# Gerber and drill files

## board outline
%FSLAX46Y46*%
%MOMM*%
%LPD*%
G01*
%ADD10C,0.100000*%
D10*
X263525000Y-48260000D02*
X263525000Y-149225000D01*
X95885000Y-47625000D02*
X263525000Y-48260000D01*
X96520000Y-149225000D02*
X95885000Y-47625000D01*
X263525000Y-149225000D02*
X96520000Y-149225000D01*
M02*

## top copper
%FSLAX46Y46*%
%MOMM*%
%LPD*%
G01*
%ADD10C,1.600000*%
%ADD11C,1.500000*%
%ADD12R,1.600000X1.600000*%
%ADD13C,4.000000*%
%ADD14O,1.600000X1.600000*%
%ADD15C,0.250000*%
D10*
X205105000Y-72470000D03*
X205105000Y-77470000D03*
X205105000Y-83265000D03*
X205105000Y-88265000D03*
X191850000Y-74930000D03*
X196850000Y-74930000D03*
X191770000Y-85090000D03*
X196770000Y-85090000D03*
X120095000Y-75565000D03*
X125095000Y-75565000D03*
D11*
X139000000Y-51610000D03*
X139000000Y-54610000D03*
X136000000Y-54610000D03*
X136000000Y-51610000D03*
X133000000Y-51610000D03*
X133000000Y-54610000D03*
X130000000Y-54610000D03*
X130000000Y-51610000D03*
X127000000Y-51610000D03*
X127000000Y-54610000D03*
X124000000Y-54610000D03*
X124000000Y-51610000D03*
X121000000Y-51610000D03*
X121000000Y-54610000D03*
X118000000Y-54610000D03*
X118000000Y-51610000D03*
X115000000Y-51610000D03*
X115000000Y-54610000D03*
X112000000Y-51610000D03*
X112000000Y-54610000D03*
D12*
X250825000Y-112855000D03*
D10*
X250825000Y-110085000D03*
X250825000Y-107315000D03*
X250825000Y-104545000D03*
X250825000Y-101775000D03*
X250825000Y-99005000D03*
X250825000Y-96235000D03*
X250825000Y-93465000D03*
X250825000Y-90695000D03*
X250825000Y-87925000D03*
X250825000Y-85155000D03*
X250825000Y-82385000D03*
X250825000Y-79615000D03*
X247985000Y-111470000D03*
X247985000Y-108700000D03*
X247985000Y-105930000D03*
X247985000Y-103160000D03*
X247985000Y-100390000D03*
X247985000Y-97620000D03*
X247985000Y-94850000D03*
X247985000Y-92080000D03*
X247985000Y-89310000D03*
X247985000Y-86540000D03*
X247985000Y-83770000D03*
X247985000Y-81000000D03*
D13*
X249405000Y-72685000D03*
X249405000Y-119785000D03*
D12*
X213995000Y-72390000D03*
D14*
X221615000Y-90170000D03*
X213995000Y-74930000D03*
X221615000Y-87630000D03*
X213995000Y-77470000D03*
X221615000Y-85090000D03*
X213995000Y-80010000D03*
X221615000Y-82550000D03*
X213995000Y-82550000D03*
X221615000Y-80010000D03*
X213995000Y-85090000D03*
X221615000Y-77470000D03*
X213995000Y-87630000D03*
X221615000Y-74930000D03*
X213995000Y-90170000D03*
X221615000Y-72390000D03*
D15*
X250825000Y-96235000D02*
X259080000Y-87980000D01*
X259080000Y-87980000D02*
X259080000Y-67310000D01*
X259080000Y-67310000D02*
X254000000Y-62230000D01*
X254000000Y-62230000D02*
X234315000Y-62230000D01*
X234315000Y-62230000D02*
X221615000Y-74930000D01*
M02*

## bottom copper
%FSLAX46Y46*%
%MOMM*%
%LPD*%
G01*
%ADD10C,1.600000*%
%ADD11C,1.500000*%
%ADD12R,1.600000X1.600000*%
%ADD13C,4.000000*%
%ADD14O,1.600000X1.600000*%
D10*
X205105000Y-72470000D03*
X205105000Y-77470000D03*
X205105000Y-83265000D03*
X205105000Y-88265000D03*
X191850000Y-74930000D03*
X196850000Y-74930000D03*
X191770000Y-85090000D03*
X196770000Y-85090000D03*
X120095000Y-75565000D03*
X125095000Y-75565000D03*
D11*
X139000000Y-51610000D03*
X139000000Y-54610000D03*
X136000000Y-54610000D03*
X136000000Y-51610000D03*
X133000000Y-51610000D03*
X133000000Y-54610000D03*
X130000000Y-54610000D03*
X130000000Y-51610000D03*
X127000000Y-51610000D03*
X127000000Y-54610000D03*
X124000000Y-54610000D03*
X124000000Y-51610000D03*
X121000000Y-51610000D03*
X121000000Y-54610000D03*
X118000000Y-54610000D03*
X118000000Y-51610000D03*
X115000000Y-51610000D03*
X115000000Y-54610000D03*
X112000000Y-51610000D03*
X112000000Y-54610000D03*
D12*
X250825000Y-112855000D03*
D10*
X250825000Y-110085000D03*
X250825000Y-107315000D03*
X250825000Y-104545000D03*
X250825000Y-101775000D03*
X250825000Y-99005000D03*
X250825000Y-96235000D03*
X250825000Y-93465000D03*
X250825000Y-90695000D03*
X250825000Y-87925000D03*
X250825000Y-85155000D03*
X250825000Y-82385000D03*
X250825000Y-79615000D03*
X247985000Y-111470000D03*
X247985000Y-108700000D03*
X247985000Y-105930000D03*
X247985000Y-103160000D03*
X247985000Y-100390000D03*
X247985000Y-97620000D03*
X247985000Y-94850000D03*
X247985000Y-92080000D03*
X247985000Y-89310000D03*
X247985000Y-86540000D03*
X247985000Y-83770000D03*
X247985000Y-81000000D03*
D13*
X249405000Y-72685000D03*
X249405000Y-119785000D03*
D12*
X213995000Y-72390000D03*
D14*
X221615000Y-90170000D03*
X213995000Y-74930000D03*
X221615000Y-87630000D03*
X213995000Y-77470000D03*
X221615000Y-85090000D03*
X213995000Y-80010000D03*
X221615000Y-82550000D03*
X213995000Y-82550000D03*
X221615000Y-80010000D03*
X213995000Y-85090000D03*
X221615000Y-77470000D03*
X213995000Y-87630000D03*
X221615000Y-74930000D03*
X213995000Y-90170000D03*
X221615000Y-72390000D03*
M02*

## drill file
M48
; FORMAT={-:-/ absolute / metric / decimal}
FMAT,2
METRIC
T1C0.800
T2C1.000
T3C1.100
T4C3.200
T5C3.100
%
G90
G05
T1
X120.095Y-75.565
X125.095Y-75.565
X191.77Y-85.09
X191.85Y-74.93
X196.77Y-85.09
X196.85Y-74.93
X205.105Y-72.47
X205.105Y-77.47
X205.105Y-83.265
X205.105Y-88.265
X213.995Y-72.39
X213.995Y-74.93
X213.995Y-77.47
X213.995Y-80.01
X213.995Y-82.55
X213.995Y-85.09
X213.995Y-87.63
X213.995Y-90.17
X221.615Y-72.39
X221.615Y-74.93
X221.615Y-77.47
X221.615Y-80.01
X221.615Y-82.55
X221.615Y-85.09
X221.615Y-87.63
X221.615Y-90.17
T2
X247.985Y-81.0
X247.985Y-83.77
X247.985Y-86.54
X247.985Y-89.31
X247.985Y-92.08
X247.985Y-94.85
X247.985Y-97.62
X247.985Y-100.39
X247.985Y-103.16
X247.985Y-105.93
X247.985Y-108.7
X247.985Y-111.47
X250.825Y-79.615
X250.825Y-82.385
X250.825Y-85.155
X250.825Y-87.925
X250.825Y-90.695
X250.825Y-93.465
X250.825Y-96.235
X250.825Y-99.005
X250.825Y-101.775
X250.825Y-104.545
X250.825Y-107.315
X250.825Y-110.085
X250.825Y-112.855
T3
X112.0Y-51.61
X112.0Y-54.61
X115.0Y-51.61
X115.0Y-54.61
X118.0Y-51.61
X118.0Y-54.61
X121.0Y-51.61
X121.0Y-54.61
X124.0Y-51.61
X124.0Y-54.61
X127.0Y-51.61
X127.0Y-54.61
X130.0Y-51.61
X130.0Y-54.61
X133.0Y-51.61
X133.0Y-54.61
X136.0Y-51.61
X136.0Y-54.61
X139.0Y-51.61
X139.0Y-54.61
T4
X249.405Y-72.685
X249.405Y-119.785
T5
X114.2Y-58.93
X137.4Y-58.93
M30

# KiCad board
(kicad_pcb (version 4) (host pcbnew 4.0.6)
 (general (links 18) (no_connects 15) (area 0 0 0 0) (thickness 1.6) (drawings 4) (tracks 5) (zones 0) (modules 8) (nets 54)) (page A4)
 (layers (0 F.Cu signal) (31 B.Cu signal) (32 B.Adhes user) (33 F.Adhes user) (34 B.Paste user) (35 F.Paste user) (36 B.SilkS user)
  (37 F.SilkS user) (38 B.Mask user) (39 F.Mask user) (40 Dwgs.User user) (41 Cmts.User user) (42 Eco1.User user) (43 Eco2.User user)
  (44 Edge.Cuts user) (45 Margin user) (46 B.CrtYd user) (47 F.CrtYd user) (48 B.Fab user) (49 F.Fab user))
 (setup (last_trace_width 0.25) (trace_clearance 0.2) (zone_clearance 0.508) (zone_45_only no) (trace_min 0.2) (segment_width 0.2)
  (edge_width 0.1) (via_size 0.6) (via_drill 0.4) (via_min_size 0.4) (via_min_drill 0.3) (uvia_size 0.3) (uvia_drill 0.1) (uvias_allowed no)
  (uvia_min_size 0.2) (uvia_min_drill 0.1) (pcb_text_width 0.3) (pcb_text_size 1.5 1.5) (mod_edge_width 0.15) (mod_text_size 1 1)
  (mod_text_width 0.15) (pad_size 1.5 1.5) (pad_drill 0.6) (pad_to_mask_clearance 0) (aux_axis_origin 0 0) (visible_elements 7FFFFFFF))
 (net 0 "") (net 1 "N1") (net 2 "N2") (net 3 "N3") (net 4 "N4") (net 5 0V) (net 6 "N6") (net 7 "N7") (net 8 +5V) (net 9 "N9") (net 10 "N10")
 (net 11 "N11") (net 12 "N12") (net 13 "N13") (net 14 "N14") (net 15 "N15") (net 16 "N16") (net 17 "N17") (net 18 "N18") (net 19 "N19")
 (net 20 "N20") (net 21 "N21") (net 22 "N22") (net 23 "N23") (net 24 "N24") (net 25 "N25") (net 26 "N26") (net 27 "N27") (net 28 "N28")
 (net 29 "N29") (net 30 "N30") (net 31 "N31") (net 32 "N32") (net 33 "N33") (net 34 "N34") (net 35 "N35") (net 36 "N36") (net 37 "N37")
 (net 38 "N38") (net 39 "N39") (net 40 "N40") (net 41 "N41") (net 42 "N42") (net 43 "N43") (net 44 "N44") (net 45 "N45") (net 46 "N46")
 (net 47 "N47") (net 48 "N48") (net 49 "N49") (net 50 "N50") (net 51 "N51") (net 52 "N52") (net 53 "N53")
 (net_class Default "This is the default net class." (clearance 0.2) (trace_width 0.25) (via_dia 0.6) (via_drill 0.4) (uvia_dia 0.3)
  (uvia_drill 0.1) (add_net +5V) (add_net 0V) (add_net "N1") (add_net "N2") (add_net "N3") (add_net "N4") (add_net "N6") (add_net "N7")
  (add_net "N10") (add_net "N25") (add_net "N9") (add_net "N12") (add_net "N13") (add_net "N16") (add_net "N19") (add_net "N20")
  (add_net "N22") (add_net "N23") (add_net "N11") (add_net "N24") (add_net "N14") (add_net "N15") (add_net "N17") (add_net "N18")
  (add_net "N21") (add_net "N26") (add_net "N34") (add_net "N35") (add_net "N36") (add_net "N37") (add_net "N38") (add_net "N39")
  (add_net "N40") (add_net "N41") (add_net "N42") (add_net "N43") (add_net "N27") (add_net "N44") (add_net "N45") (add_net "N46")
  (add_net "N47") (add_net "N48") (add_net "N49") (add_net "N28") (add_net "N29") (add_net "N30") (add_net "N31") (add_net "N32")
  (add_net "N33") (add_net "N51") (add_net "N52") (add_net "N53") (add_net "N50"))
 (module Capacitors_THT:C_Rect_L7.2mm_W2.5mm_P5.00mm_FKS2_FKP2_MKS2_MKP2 (layer F.Cu) (at 205.105 72.47 270)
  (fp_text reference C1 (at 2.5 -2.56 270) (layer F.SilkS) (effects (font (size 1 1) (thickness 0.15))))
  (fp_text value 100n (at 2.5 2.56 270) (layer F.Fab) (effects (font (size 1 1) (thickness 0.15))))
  (pad 1 thru_hole circle (at 0 0 270) (size 1.6 1.6) (drill 0.8) (layers *.Cu *.Mask) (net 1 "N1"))
  (pad 2 thru_hole circle (at 5 0 270) (size 1.6 1.6) (drill 0.8) (layers *.Cu *.Mask) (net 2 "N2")))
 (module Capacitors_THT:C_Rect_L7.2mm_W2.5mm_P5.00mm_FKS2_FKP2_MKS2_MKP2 (layer F.Cu) (at 205.105 83.265 270)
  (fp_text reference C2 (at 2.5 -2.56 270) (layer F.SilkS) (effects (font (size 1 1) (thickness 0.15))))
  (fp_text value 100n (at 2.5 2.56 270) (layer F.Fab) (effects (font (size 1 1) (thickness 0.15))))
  (pad 1 thru_hole circle (at 0 0 270) (size 1.6 1.6) (drill 0.8) (layers *.Cu *.Mask) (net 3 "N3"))
  (pad 2 thru_hole circle (at 5 0 270) (size 1.6 1.6) (drill 0.8) (layers *.Cu *.Mask) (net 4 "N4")))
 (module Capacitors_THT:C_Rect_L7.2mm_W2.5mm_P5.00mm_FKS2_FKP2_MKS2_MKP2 (layer F.Cu) (at 191.85 74.93)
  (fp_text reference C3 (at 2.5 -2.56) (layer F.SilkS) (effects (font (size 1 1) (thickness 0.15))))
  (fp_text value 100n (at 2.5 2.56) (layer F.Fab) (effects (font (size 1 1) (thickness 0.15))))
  (pad 1 thru_hole circle (at 0 0) (size 1.6 1.6) (drill 0.8) (layers *.Cu *.Mask) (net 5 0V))
  (pad 2 thru_hole circle (at 5 0) (size 1.6 1.6) (drill 0.8) (layers *.Cu *.Mask) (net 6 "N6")))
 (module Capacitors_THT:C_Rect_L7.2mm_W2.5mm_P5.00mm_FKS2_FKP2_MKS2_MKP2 (layer F.Cu) (at 191.77 85.09)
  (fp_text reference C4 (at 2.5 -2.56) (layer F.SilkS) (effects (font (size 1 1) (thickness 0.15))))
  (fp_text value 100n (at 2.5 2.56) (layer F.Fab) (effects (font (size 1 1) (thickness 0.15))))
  (pad 1 thru_hole circle (at 0 0) (size 1.6 1.6) (drill 0.8) (layers *.Cu *.Mask) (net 5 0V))
  (pad 2 thru_hole circle (at 5 0) (size 1.6 1.6) (drill 0.8) (layers *.Cu *.Mask) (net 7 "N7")))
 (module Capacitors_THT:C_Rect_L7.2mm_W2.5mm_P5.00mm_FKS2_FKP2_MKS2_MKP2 (layer F.Cu) (at 120.095 75.565)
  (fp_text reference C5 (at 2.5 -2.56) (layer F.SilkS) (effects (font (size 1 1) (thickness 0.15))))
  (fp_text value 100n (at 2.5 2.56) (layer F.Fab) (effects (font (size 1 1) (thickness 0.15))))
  (pad 1 thru_hole circle (at 0 0) (size 1.6 1.6) (drill 0.8) (layers *.Cu *.Mask) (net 5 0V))
  (pad 2 thru_hole circle (at 5 0) (size 1.6 1.6) (drill 0.8) (layers *.Cu *.Mask) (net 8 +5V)))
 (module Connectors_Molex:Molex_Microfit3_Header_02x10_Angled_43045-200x (layer F.Cu) (at 139 54.61)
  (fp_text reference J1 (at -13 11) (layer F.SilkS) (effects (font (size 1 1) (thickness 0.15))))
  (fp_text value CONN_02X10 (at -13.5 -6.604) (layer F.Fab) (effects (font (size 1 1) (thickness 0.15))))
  (pad 11 thru_hole circle (at 0 -3) (size 1.5 1.5) (drill 1.1) (layers *.Cu *.Mask) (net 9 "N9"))
  (pad 1 thru_hole circle (at 0 0) (size 1.5 1.5) (drill 1.1) (layers *.Cu *.Mask) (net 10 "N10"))
  (pad 2 thru_hole circle (at -3 0) (size 1.5 1.5) (drill 1.1) (layers *.Cu *.Mask) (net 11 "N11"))
  (pad 12 thru_hole circle (at -3 -3) (size 1.5 1.5) (drill 1.1) (layers *.Cu *.Mask) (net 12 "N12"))
  (pad 13 thru_hole circle (at -6 -3) (size 1.5 1.5) (drill 1.1) (layers *.Cu *.Mask) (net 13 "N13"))
  (pad 3 thru_hole circle (at -6 0) (size 1.5 1.5) (drill 1.1) (layers *.Cu *.Mask) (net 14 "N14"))
  (pad 4 thru_hole circle (at -9 0) (size 1.5 1.5) (drill 1.1) (layers *.Cu *.Mask) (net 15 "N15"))
  (pad 14 thru_hole circle (at -9 -3) (size 1.5 1.5) (drill 1.1) (layers *.Cu *.Mask) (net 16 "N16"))
  (pad 15 thru_hole circle (at -12 -3) (size 1.5 1.5) (drill 1.1) (layers *.Cu *.Mask) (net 5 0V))
  (pad 5 thru_hole circle (at -12 0) (size 1.5 1.5) (drill 1.1) (layers *.Cu *.Mask) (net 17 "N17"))
  (pad 6 thru_hole circle (at -15 0) (size 1.5 1.5) (drill 1.1) (layers *.Cu *.Mask) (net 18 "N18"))
  (pad 16 thru_hole circle (at -15 -3) (size 1.5 1.5) (drill 1.1) (layers *.Cu *.Mask) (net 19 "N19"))
  (pad "" np_thru_hole circle (at -1.6 4.32) (size 3.1 3.1) (drill 3.1) (layers *.Cu *.Mask))
  (pad 17 thru_hole circle (at -18 -3) (size 1.5 1.5) (drill 1.1) (layers *.Cu *.Mask) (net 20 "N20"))
  (pad 7 thru_hole circle (at -18 0) (size 1.5 1.5) (drill 1.1) (layers *.Cu *.Mask) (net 8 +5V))
  (pad 8 thru_hole circle (at -21 0) (size 1.5 1.5) (drill 1.1) (layers *.Cu *.Mask) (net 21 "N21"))
  (pad 18 thru_hole circle (at -21 -3) (size 1.5 1.5) (drill 1.1) (layers *.Cu *.Mask) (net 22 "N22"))
  (pad 19 thru_hole circle (at -24 -3) (size 1.5 1.5) (drill 1.1) (layers *.Cu *.Mask) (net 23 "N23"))
  (pad 9 thru_hole circle (at -24 0) (size 1.5 1.5) (drill 1.1) (layers *.Cu *.Mask) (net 5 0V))
  (pad 20 thru_hole circle (at -27 -3) (size 1.5 1.5) (drill 1.1) (layers *.Cu *.Mask) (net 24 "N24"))
  (pad 10 thru_hole circle (at -27 0) (size 1.5 1.5) (drill 1.1) (layers *.Cu *.Mask) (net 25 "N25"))
  (pad "" np_thru_hole circle (at -24.8 4.32) (size 3.1 3.1) (drill 3.1) (layers *.Cu *.Mask)))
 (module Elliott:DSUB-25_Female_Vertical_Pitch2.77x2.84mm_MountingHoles (layer F.Cu) (at 250.825 112.855 270)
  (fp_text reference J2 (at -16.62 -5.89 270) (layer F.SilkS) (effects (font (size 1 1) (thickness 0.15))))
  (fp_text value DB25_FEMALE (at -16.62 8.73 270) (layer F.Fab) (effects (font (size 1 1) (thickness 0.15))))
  (pad 1 thru_hole rect (at 0 0 270) (size 1.6 1.6) (drill 1) (layers *.Cu *.Mask) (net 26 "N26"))
  (pad 2 thru_hole circle (at -2.77 0 270) (size 1.6 1.6) (drill 1) (layers *.Cu *.Mask) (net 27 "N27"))
  (pad 3 thru_hole circle (at -5.54 0 270) (size 1.6 1.6) (drill 1) (layers *.Cu *.Mask) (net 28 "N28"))
  (pad 4 thru_hole circle (at -8.31 0 270) (size 1.6 1.6) (drill 1) (layers *.Cu *.Mask) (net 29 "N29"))
  (pad 5 thru_hole circle (at -11.08 0 270) (size 1.6 1.6) (drill 1) (layers *.Cu *.Mask) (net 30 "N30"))
  (pad 6 thru_hole circle (at -13.85 0 270) (size 1.6 1.6) (drill 1) (layers *.Cu *.Mask) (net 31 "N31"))
  (pad 7 thru_hole circle (at -16.62 0 270) (size 1.6 1.6) (drill 1) (layers *.Cu *.Mask) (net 5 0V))
  (pad 8 thru_hole circle (at -19.39 0 270) (size 1.6 1.6) (drill 1) (layers *.Cu *.Mask) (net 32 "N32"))
  (pad 9 thru_hole circle (at -22.16 0 270) (size 1.6 1.6) (drill 1) (layers *.Cu *.Mask) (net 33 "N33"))
  (pad 10 thru_hole circle (at -24.93 0 270) (size 1.6 1.6) (drill 1) (layers *.Cu *.Mask) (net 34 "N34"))
  (pad 11 thru_hole circle (at -27.7 0 270) (size 1.6 1.6) (drill 1) (layers *.Cu *.Mask) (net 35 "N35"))
  (pad 12 thru_hole circle (at -30.47 0 270) (size 1.6 1.6) (drill 1) (layers *.Cu *.Mask) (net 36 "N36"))
  (pad 13 thru_hole circle (at -33.24 0 270) (size 1.6 1.6) (drill 1) (layers *.Cu *.Mask) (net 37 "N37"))
  (pad 14 thru_hole circle (at -1.385 2.84 270) (size 1.6 1.6) (drill 1) (layers *.Cu *.Mask) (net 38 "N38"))
  (pad 15 thru_hole circle (at -4.155 2.84 270) (size 1.6 1.6) (drill 1) (layers *.Cu *.Mask) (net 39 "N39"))
  (pad 16 thru_hole circle (at -6.925 2.84 270) (size 1.6 1.6) (drill 1) (layers *.Cu *.Mask) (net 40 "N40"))
  (pad 17 thru_hole circle (at -9.695 2.84 270) (size 1.6 1.6) (drill 1) (layers *.Cu *.Mask) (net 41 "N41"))
  (pad 18 thru_hole circle (at -12.465 2.84 270) (size 1.6 1.6) (drill 1) (layers *.Cu *.Mask) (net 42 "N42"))
  (pad 19 thru_hole circle (at -15.235 2.84 270) (size 1.6 1.6) (drill 1) (layers *.Cu *.Mask) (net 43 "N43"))
  (pad 20 thru_hole circle (at -18.005 2.84 270) (size 1.6 1.6) (drill 1) (layers *.Cu *.Mask) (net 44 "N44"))
  (pad 21 thru_hole circle (at -20.775 2.84 270) (size 1.6 1.6) (drill 1) (layers *.Cu *.Mask) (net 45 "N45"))
  (pad 22 thru_hole circle (at -23.545 2.84 270) (size 1.6 1.6) (drill 1) (layers *.Cu *.Mask) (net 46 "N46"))
  (pad 23 thru_hole circle (at -26.315 2.84 270) (size 1.6 1.6) (drill 1) (layers *.Cu *.Mask) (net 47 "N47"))
  (pad 24 thru_hole circle (at -29.085 2.84 270) (size 1.6 1.6) (drill 1) (layers *.Cu *.Mask) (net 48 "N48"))
  (pad 25 thru_hole circle (at -31.855 2.84 270) (size 1.6 1.6) (drill 1) (layers *.Cu *.Mask) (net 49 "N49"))
  (pad 0 thru_hole circle (at -40.17 1.42 270) (size 4 4) (drill 3.2) (layers *.Cu *.Mask))
  (pad 0 thru_hole circle (at 6.93 1.42 270) (size 4 4) (drill 3.2) (layers *.Cu *.Mask)))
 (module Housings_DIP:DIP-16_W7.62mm (layer F.Cu) (at 213.995 72.39)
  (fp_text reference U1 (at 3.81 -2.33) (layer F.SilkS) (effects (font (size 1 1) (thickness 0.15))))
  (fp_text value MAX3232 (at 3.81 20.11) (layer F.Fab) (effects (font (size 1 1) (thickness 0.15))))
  (pad 1 thru_hole rect (at 0 0) (size 1.6 1.6) (drill 0.8) (layers *.Cu *.Mask) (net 1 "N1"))
  (pad 9 thru_hole oval (at 7.62 17.78) (size 1.6 1.6) (drill 0.8) (layers *.Cu *.Mask) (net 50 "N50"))
  (pad 2 thru_hole oval (at 0 2.54) (size 1.6 1.6) (drill 0.8) (layers *.Cu *.Mask) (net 6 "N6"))
  (pad 10 thru_hole oval (at 7.62 15.24) (size 1.6 1.6) (drill 0.8) (layers *.Cu *.Mask) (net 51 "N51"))
  (pad 3 thru_hole oval (at 0 5.08) (size 1.6 1.6) (drill 0.8) (layers *.Cu *.Mask) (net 2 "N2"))
  (pad 11 thru_hole oval (at 7.62 12.7) (size 1.6 1.6) (drill 0.8) (layers *.Cu *.Mask) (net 23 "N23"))
  (pad 4 thru_hole oval (at 0 7.62) (size 1.6 1.6) (drill 0.8) (layers *.Cu *.Mask) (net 3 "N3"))
  (pad 12 thru_hole oval (at 7.62 10.16) (size 1.6 1.6) (drill 0.8) (layers *.Cu *.Mask) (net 20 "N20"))
  (pad 5 thru_hole oval (at 0 10.16) (size 1.6 1.6) (drill 0.8) (layers *.Cu *.Mask) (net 4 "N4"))
  (pad 13 thru_hole oval (at 7.62 7.62) (size 1.6 1.6) (drill 0.8) (layers *.Cu *.Mask) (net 28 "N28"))
  (pad 6 thru_hole oval (at 0 12.7) (size 1.6 1.6) (drill 0.8) (layers *.Cu *.Mask) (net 7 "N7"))
  (pad 14 thru_hole oval (at 7.62 5.08) (size 1.6 1.6) (drill 0.8) (layers *.Cu *.Mask) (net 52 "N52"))
  (pad 7 thru_hole oval (at 0 15.24) (size 1.6 1.6) (drill 0.8) (layers *.Cu *.Mask) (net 27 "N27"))
  (pad 15 thru_hole oval (at 7.62 2.54) (size 1.6 1.6) (drill 0.8) (layers *.Cu *.Mask) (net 5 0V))
  (pad 8 thru_hole oval (at 0 17.78) (size 1.6 1.6) (drill 0.8) (layers *.Cu *.Mask) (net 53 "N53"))
  (pad 16 thru_hole oval (at 7.62 0) (size 1.6 1.6) (drill 0.8) (layers *.Cu *.Mask) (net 8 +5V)))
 (gr_line (start 263.525 48.26) (end 263.525 149.225) (layer Edge.Cuts) (width 0.1))
 (gr_line (start 95.885 47.625) (end 263.525 48.26) (layer Edge.Cuts) (width 0.1))
 (gr_line (start 96.52 149.225) (end 95.885 47.625) (layer Edge.Cuts) (width 0.1))
 (gr_line (start 263.525 149.225) (end 96.52 149.225) (layer Edge.Cuts) (width 0.1))
 (segment (start 250.825 96.235) (end 259.08 87.98) (width 0.25) (layer F.Cu) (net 5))
 (segment (start 259.08 87.98) (end 259.08 67.31) (width 0.25) (layer F.Cu) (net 5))
 (segment (start 259.08 67.31) (end 254 62.23) (width 0.25) (layer F.Cu) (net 5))
 (segment (start 254 62.23) (end 234.315 62.23) (width 0.25) (layer F.Cu) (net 5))
 (segment (start 234.315 62.23) (end 221.615 74.93) (width 0.25) (layer F.Cu) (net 5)))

